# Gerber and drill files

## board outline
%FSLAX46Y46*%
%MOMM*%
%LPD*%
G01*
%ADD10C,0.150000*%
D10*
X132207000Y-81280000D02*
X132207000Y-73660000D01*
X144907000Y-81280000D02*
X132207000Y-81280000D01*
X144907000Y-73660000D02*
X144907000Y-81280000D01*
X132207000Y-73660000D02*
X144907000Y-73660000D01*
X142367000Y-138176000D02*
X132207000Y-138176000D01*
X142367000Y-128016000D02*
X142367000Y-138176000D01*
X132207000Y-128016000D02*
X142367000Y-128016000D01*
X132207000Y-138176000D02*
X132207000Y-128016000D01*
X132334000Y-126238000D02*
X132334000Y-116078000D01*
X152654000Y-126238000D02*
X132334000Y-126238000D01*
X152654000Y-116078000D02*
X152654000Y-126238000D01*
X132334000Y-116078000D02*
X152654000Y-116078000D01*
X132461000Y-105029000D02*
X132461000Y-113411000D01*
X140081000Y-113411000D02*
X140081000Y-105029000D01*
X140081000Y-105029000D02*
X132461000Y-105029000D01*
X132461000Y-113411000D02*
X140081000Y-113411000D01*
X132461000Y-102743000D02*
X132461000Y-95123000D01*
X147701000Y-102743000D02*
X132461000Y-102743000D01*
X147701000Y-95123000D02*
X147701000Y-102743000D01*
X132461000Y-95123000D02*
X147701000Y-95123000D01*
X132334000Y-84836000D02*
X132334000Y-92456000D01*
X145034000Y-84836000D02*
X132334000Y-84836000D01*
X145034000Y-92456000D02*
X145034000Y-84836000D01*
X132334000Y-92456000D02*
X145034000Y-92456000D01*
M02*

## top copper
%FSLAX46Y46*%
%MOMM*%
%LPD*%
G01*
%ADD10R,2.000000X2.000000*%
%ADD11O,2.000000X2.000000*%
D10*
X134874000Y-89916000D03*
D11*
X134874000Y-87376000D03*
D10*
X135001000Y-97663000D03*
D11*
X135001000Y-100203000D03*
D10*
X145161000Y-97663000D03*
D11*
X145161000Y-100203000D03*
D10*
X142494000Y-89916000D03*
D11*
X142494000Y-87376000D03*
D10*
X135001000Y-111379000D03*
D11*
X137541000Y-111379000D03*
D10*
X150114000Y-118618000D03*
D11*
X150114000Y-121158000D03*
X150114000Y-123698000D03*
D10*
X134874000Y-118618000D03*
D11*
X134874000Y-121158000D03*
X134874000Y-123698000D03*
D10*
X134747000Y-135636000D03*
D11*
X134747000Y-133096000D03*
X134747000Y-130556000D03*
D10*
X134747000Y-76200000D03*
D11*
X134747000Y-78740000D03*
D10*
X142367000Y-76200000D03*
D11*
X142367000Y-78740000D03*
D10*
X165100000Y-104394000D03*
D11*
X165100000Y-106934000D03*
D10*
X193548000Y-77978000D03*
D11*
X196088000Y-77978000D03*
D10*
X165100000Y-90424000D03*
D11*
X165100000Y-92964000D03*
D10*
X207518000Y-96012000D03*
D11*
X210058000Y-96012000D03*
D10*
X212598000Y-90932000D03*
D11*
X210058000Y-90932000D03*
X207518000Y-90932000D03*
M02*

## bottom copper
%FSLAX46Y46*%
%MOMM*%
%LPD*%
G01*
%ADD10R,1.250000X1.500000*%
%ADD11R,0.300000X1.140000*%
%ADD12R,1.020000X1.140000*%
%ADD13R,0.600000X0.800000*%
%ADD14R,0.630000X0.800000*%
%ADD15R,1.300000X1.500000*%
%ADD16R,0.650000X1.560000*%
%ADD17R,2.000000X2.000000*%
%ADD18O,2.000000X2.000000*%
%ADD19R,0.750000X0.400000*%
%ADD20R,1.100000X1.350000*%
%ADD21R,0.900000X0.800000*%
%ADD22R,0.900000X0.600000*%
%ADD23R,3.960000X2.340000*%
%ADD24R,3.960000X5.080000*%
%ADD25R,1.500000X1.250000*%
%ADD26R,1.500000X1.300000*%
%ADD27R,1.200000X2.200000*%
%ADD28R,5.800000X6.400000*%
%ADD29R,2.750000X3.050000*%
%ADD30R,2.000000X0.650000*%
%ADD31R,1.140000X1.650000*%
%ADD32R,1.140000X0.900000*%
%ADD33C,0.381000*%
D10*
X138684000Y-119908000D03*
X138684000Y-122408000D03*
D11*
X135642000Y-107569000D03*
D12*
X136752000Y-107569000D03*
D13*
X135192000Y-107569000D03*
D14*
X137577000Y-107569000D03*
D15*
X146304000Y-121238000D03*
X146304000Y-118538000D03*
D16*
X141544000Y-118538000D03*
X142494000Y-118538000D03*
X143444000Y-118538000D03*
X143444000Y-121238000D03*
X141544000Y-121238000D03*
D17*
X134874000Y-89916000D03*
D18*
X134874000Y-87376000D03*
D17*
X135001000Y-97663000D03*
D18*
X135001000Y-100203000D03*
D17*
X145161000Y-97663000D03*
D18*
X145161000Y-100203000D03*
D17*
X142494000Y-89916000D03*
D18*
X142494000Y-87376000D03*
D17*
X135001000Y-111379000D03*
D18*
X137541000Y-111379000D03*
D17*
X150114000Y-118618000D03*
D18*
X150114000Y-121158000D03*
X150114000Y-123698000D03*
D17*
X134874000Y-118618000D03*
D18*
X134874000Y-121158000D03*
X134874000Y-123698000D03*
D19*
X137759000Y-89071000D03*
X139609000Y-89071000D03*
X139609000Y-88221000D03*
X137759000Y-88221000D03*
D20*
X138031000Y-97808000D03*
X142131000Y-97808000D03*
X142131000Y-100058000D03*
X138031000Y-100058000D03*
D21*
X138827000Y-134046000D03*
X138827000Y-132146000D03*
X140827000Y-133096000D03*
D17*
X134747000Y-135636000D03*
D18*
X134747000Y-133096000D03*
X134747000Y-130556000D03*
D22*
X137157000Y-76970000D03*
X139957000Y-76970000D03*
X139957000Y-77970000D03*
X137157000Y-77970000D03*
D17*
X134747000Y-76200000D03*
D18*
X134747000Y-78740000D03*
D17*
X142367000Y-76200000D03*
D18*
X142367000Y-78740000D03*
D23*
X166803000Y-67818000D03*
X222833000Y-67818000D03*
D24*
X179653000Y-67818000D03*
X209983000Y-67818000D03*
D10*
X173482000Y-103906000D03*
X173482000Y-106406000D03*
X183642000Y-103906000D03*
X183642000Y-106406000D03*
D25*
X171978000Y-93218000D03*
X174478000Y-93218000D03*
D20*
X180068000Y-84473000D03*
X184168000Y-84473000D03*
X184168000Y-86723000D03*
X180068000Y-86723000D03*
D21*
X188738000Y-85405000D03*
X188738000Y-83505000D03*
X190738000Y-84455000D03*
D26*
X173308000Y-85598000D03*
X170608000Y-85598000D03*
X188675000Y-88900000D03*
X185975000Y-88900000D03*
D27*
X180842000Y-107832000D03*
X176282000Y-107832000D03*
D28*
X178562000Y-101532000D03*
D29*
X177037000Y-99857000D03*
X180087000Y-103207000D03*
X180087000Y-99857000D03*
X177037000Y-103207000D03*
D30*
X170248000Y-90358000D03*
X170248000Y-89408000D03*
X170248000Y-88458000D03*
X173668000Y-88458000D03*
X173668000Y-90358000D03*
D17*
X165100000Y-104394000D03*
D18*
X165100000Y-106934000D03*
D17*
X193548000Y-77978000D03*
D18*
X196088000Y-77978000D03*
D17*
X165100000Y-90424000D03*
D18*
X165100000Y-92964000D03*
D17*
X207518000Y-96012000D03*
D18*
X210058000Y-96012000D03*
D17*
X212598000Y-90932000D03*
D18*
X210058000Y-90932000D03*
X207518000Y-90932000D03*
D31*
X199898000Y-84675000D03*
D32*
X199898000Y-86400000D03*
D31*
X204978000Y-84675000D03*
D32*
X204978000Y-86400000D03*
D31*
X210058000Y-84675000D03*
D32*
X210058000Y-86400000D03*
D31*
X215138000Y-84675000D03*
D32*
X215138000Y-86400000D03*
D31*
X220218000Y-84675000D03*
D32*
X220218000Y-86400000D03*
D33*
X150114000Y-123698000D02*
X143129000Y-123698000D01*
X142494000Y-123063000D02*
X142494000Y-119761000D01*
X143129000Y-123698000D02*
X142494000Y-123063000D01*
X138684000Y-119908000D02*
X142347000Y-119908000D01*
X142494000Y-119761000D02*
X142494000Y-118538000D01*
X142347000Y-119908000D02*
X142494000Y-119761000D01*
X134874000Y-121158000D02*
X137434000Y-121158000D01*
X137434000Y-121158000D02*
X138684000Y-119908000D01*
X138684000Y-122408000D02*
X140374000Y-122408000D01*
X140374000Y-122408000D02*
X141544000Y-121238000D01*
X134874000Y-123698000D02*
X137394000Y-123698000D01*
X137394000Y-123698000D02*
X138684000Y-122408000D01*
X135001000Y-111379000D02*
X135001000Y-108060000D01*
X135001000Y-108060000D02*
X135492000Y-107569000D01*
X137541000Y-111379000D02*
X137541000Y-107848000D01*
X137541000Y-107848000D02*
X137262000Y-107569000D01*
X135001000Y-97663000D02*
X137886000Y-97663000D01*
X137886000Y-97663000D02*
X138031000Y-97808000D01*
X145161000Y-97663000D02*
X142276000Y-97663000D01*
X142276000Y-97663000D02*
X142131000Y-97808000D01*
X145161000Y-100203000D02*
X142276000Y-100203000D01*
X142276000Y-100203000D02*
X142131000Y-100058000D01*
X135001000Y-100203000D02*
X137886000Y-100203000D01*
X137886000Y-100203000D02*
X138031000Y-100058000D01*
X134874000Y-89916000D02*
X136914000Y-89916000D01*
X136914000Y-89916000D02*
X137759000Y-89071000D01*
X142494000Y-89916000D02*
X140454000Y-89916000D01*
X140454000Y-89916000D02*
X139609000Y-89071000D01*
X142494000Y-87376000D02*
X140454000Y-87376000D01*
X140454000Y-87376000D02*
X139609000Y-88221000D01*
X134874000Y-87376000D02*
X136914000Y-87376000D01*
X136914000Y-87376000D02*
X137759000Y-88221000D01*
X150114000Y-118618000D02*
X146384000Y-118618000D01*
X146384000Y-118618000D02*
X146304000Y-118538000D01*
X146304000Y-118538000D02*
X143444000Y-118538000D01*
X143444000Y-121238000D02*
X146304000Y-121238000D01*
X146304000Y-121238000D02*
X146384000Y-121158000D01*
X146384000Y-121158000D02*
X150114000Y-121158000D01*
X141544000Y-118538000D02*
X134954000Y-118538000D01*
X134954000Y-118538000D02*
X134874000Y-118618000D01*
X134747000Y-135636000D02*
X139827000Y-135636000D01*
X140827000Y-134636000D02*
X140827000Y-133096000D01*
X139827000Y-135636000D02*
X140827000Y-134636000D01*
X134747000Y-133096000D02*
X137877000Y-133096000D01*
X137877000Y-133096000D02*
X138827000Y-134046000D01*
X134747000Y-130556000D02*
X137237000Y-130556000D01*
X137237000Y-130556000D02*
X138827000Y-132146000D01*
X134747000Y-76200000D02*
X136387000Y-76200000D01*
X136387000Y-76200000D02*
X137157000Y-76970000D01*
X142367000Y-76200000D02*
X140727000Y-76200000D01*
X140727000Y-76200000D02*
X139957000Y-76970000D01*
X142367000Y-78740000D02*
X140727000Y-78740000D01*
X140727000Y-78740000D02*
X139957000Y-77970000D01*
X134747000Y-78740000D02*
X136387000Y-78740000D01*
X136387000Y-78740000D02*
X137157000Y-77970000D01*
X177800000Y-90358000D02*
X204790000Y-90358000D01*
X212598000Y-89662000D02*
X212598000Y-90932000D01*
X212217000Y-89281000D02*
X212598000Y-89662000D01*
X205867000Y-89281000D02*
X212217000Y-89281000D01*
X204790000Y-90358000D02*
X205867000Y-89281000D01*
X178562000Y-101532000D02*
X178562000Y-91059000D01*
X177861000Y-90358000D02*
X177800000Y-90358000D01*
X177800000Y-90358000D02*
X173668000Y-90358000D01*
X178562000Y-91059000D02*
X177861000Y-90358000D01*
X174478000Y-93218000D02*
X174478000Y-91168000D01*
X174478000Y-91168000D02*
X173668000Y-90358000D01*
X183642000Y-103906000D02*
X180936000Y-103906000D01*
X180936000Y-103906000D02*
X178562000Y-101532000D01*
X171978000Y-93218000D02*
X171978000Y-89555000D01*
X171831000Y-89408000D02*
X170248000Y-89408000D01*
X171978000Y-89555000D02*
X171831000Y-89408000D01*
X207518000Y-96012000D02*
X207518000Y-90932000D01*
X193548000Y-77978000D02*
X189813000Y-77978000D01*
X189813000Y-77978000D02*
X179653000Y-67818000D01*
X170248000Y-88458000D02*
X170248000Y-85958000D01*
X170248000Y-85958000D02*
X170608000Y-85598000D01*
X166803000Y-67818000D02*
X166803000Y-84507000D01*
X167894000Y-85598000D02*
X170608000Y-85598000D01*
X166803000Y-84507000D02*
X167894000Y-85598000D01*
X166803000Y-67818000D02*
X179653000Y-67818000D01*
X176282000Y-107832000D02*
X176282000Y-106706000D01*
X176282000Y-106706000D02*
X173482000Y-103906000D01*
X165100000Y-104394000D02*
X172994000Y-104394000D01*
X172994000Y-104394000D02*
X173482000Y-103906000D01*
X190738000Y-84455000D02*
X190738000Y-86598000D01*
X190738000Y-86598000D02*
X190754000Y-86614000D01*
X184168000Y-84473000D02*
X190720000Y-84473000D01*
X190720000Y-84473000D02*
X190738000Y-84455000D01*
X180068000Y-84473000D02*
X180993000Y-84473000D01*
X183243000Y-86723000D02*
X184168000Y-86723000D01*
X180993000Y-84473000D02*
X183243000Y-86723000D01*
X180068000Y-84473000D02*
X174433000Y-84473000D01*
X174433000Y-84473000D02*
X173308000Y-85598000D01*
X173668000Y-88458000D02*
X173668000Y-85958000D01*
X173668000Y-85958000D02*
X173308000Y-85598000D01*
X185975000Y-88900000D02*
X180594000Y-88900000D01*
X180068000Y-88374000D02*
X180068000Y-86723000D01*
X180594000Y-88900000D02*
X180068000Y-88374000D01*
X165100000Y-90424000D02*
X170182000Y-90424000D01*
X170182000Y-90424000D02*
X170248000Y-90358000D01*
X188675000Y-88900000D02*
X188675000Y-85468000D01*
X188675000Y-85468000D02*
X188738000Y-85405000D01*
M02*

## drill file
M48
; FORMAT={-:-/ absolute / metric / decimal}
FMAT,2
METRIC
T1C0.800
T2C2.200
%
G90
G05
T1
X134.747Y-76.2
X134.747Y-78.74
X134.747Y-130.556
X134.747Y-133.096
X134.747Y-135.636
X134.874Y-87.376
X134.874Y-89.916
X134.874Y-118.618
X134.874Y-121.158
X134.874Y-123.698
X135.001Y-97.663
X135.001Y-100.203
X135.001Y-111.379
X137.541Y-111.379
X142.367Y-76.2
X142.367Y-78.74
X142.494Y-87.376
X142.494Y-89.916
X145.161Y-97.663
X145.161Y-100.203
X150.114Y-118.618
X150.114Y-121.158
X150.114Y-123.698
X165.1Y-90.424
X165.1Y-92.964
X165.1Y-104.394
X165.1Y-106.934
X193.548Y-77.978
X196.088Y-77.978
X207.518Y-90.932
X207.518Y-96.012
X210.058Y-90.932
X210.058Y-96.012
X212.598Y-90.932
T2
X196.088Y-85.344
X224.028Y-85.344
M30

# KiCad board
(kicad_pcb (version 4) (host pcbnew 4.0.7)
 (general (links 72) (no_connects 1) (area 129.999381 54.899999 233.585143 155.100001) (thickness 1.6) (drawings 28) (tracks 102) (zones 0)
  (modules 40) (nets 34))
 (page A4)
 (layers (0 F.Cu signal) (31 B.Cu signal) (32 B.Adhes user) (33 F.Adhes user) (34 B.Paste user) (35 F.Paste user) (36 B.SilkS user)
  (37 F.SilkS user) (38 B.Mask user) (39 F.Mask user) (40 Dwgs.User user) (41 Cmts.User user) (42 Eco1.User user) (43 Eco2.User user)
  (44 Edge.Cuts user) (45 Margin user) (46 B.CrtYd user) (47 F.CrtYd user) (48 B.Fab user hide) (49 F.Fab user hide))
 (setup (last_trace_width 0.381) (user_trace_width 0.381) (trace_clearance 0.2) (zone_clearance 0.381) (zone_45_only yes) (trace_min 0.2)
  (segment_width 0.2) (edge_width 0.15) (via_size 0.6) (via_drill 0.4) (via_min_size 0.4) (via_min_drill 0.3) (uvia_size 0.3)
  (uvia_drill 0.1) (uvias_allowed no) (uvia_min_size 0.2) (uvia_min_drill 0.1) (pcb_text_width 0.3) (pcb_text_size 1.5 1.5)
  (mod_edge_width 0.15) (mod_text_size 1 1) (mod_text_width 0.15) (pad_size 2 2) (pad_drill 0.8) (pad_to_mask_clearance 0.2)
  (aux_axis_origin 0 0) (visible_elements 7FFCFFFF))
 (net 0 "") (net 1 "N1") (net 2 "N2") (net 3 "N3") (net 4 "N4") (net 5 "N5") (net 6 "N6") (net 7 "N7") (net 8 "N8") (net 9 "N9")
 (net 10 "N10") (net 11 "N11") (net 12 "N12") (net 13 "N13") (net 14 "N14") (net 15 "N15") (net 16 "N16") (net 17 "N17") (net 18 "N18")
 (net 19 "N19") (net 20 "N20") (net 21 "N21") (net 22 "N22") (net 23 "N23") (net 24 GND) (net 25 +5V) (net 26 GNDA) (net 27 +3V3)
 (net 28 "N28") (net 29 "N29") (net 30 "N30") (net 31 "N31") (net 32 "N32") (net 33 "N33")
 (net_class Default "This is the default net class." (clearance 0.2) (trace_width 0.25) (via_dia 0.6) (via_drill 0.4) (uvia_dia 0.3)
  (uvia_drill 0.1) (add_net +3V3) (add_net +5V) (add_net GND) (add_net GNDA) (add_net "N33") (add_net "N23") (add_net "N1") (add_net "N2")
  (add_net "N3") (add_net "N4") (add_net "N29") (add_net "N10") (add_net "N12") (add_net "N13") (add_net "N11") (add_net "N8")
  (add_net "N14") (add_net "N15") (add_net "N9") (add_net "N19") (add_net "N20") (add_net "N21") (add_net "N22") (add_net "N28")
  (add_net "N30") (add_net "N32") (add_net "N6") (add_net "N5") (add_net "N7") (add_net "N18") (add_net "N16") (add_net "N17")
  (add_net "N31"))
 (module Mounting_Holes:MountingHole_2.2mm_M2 (layer F.Cu) (at 224.028 85.344)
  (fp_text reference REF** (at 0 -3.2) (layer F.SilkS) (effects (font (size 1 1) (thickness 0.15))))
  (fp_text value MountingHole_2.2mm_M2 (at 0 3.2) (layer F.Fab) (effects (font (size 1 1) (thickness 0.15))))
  (pad 1 np_thru_hole circle (at 0 0) (size 2.2 2.2) (drill 2.2) (layers *.Cu *.Mask)))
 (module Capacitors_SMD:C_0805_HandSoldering (layer B.Cu) (at 138.684 121.158 270)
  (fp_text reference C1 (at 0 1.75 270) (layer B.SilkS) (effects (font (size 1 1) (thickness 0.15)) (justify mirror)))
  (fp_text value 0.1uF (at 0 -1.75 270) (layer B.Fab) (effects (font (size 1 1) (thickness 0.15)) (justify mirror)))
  (pad 1 smd rect (at -1.25 0 270) (size 1.5 1.25) (layers B.Cu B.Paste B.Mask) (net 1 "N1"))
  (pad 2 smd rect (at 1.25 0 270) (size 1.5 1.25) (layers B.Cu B.Paste B.Mask) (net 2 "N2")))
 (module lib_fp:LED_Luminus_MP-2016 (layer B.Cu) (at 136.017 107.569)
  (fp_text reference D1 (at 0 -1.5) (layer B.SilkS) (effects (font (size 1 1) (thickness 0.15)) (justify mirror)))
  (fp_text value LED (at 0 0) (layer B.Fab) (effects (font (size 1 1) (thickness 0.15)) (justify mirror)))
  (pad 1 smd rect (at -0.225 0) (size 0.3 1.14) (drill (offset -0.15 0)) (layers B.Cu B.Paste B.Mask) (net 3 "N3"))
  (pad 2 smd rect (at 0.225 0) (size 1.02 1.14) (drill (offset 0.51 0)) (layers B.Cu B.Paste B.Mask) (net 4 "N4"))
  (pad 1 smd rect (at -0.525 0) (size 0.6 0.8) (drill (offset -0.3 0)) (layers B.Cu B.Paste B.Mask) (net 3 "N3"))
  (pad 2 smd rect (at 1.245 0) (size 0.63 0.8) (drill (offset 0.315 0)) (layers B.Cu B.Paste B.Mask) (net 4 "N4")))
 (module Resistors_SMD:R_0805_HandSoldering (layer B.Cu) (at 146.304 119.888 90)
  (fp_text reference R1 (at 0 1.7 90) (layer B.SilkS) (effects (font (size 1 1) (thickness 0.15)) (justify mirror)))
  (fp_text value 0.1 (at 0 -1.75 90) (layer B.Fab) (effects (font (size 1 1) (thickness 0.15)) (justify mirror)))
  (pad 1 smd rect (at -1.35 0 90) (size 1.5 1.3) (layers B.Cu B.Paste B.Mask) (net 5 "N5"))
  (pad 2 smd rect (at 1.35 0 90) (size 1.5 1.3) (layers B.Cu B.Paste B.Mask) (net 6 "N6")))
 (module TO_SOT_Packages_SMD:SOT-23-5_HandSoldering (layer B.Cu) (at 142.494 119.888 270)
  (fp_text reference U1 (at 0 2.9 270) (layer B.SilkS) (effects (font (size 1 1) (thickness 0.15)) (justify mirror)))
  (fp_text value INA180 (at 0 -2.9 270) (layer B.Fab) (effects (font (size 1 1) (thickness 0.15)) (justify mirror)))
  (pad 1 smd rect (at -1.35 0.95 270) (size 1.56 0.65) (layers B.Cu B.Paste B.Mask) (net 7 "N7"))
  (pad 2 smd rect (at -1.35 0 270) (size 1.56 0.65) (layers B.Cu B.Paste B.Mask) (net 1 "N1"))
  (pad 3 smd rect (at -1.35 -0.95 270) (size 1.56 0.65) (layers B.Cu B.Paste B.Mask) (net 6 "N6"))
  (pad 4 smd rect (at 1.35 -0.95 270) (size 1.56 0.65) (layers B.Cu B.Paste B.Mask) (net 5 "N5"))
  (pad 5 smd rect (at 1.35 0.95 270) (size 1.56 0.65) (layers B.Cu B.Paste B.Mask) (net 2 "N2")))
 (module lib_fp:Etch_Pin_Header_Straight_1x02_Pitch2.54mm (layer F.Cu) (at 134.874 89.916 180)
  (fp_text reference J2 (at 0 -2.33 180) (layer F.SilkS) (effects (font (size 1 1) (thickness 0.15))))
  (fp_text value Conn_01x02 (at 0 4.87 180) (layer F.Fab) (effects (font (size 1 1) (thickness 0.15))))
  (pad 1 thru_hole rect (at 0 0 180) (size 2 2) (drill 0.8) (layers *.Cu *.Mask) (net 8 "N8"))
  (pad 2 thru_hole oval (at 0 2.54 180) (size 2 2) (drill 0.8) (layers *.Cu *.Mask) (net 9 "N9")))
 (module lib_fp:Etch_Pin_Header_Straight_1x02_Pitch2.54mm (layer F.Cu) (at 135.001 97.663)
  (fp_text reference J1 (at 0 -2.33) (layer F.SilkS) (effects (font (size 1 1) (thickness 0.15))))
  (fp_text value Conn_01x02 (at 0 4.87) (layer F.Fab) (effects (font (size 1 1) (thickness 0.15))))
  (pad 1 thru_hole rect (at 0 0) (size 2 2) (drill 0.8) (layers *.Cu *.Mask) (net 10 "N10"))
  (pad 2 thru_hole oval (at 0 2.54) (size 2 2) (drill 0.8) (layers *.Cu *.Mask) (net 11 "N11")))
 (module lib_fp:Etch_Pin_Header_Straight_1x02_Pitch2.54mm (layer F.Cu) (at 145.161 97.663)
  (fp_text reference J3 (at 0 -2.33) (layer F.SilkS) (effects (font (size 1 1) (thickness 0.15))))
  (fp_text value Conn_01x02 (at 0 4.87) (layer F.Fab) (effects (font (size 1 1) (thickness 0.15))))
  (pad 1 thru_hole rect (at 0 0) (size 2 2) (drill 0.8) (layers *.Cu *.Mask) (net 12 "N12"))
  (pad 2 thru_hole oval (at 0 2.54) (size 2 2) (drill 0.8) (layers *.Cu *.Mask) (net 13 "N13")))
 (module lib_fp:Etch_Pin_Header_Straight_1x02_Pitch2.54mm (layer F.Cu) (at 142.494 89.916 180)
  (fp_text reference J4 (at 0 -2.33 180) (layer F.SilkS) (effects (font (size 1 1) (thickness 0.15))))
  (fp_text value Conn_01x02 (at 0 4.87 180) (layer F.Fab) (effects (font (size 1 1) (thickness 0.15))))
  (pad 1 thru_hole rect (at 0 0 180) (size 2 2) (drill 0.8) (layers *.Cu *.Mask) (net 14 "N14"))
  (pad 2 thru_hole oval (at 0 2.54 180) (size 2 2) (drill 0.8) (layers *.Cu *.Mask) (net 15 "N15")))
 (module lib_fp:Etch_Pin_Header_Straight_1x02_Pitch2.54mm (layer F.Cu) (at 135.001 111.379 90)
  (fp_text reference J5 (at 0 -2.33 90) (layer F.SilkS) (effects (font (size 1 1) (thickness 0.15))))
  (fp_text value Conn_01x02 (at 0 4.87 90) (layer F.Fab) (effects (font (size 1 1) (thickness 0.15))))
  (pad 1 thru_hole rect (at 0 0 90) (size 2 2) (drill 0.8) (layers *.Cu *.Mask) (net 3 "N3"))
  (pad 2 thru_hole oval (at 0 2.54 90) (size 2 2) (drill 0.8) (layers *.Cu *.Mask) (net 4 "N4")))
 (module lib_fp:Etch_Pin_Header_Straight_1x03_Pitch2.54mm (layer F.Cu) (at 150.114 118.618)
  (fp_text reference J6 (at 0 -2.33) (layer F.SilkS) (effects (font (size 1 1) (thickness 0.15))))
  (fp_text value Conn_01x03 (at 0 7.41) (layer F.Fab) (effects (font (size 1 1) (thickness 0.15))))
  (pad 1 thru_hole rect (at 0 0) (size 2 2) (drill 0.8) (layers *.Cu *.Mask) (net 6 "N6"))
  (pad 2 thru_hole oval (at 0 2.54) (size 2 2) (drill 0.8) (layers *.Cu *.Mask) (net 5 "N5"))
  (pad 3 thru_hole oval (at 0 5.08) (size 2 2) (drill 0.8) (layers *.Cu *.Mask) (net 1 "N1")))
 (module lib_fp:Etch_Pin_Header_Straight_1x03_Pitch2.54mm (layer F.Cu) (at 134.874 118.618)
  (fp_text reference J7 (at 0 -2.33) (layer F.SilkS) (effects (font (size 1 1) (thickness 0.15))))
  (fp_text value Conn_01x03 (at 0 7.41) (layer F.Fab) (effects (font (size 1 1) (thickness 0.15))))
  (pad 1 thru_hole rect (at 0 0) (size 2 2) (drill 0.8) (layers *.Cu *.Mask) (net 7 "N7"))
  (pad 2 thru_hole oval (at 0 2.54) (size 2 2) (drill 0.8) (layers *.Cu *.Mask) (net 1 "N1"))
  (pad 3 thru_hole oval (at 0 5.08) (size 2 2) (drill 0.8) (layers *.Cu *.Mask) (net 2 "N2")))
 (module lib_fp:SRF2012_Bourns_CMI (layer B.Cu) (at 138.684 88.646)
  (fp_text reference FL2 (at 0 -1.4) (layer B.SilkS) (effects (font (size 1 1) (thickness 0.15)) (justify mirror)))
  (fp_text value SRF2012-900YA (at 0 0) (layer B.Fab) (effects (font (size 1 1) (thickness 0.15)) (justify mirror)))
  (pad 1 smd rect (at -0.925 0.425) (size 0.75 0.4) (layers B.Cu B.Paste B.Mask) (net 8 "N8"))
  (pad 2 smd rect (at 0.925 0.425) (size 0.75 0.4) (layers B.Cu B.Paste B.Mask) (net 14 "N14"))
  (pad 3 smd rect (at 0.925 -0.425) (size 0.75 0.4) (layers B.Cu B.Paste B.Mask) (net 15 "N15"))
  (pad 4 smd rect (at -0.925 -0.425) (size 0.75 0.4) (layers B.Cu B.Paste B.Mask) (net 9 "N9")))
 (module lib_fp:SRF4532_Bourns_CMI (layer B.Cu) (at 140.081 98.933)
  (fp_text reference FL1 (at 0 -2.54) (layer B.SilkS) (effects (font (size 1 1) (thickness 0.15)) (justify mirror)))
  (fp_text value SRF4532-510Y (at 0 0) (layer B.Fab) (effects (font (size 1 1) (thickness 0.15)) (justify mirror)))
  (pad 1 smd rect (at -2.05 -1.125) (size 1.1 1.35) (layers B.Cu B.Paste B.Mask) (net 10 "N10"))
  (pad 2 smd rect (at 2.05 -1.125) (size 1.1 1.35) (layers B.Cu B.Paste B.Mask) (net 12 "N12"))
  (pad 3 smd rect (at 2.05 1.125) (size 1.1 1.35) (layers B.Cu B.Paste B.Mask) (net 13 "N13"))
  (pad 4 smd rect (at -2.05 1.125) (size 1.1 1.35) (layers B.Cu B.Paste B.Mask) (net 11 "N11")))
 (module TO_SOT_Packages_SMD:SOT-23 (layer B.Cu) (at 139.827 133.096)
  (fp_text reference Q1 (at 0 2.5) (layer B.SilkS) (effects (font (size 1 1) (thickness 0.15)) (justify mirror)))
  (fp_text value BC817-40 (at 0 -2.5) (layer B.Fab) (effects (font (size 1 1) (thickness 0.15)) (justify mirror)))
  (pad 1 smd rect (at -1 0.95) (size 0.9 0.8) (layers B.Cu B.Paste B.Mask) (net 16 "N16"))
  (pad 2 smd rect (at -1 -0.95) (size 0.9 0.8) (layers B.Cu B.Paste B.Mask) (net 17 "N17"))
  (pad 3 smd rect (at 1 0) (size 0.9 0.8) (layers B.Cu B.Paste B.Mask) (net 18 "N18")))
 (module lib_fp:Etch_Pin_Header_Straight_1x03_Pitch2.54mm (layer F.Cu) (at 134.747 135.636 180)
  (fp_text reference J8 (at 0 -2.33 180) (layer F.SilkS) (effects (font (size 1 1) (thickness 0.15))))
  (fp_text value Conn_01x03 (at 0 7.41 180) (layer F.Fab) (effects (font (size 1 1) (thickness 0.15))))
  (pad 1 thru_hole rect (at 0 0 180) (size 2 2) (drill 0.8) (layers *.Cu *.Mask) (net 18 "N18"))
  (pad 2 thru_hole oval (at 0 2.54 180) (size 2 2) (drill 0.8) (layers *.Cu *.Mask) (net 16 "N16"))
  (pad 3 thru_hole oval (at 0 5.08 180) (size 2 2) (drill 0.8) (layers *.Cu *.Mask) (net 17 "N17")))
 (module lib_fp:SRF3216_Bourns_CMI (layer B.Cu) (at 138.557 77.47)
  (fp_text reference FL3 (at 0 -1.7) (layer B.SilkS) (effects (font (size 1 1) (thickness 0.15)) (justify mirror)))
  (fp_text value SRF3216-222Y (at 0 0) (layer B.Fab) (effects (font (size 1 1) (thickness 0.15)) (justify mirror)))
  (pad 1 smd rect (at -1.4 -0.5) (size 0.9 0.6) (layers B.Cu B.Paste B.Mask) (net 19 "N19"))
  (pad 2 smd rect (at 1.4 -0.5) (size 0.9 0.6) (layers B.Cu B.Paste B.Mask) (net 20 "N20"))
  (pad 3 smd rect (at 1.4 0.5) (size 0.9 0.6) (layers B.Cu B.Paste B.Mask) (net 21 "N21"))
  (pad 4 smd rect (at -1.4 0.5) (size 0.9 0.6) (layers B.Cu B.Paste B.Mask) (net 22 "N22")))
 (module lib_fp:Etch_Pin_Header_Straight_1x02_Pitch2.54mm (layer F.Cu) (at 134.747 76.2)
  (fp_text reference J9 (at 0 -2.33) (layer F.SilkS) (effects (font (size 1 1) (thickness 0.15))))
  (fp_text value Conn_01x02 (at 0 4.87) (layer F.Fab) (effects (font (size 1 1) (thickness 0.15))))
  (pad 1 thru_hole rect (at 0 0) (size 2 2) (drill 0.8) (layers *.Cu *.Mask) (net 19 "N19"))
  (pad 2 thru_hole oval (at 0 2.54) (size 2 2) (drill 0.8) (layers *.Cu *.Mask) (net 22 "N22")))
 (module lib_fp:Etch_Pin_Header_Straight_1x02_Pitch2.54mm (layer F.Cu) (at 142.367 76.2)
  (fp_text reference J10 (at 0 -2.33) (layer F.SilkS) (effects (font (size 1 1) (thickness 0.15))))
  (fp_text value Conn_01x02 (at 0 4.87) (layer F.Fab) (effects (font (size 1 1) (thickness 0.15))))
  (pad 1 thru_hole rect (at 0 0) (size 2 2) (drill 0.8) (layers *.Cu *.Mask) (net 20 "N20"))
  (pad 2 thru_hole oval (at 0 2.54) (size 2 2) (drill 0.8) (layers *.Cu *.Mask) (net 21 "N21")))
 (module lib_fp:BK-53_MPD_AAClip (layer B.Cu) (at 194.818 67.818 270)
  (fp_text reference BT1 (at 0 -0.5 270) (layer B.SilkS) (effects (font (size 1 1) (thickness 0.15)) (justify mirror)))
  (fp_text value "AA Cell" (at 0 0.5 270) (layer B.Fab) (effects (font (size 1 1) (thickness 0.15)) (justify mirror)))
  (pad 1 smd rect (at 0 28.015 270) (size 2.34 3.96) (layers B.Cu B.Paste B.Mask) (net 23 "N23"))
  (pad 2 smd rect (at 0 -28.015 270) (size 2.34 3.96) (layers B.Cu B.Paste B.Mask) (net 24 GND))
  (pad 1 smd rect (at 0 15.165 270) (size 5.08 3.96) (layers B.Cu B.Paste B.Mask) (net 23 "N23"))
  (pad 2 smd rect (at 0 -15.165 270) (size 5.08 3.96) (layers B.Cu B.Paste B.Mask) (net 24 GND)))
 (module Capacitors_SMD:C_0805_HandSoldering (layer B.Cu) (at 173.482 105.156 270)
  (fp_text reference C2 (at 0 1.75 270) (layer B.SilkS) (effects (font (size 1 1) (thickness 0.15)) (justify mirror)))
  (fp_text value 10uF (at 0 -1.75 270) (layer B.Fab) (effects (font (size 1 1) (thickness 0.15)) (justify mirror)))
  (pad 1 smd rect (at -1.25 0 270) (size 1.5 1.25) (layers B.Cu B.Paste B.Mask) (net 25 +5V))
  (pad 2 smd rect (at 1.25 0 270) (size 1.5 1.25) (layers B.Cu B.Paste B.Mask) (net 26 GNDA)))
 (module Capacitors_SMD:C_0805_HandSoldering (layer B.Cu) (at 183.642 105.156 270)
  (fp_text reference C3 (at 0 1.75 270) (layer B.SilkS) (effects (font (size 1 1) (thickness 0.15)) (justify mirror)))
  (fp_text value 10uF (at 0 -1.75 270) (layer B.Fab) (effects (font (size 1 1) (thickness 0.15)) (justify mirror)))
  (pad 1 smd rect (at -1.25 0 270) (size 1.5 1.25) (layers B.Cu B.Paste B.Mask) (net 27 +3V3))
  (pad 2 smd rect (at 1.25 0 270) (size 1.5 1.25) (layers B.Cu B.Paste B.Mask) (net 26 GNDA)))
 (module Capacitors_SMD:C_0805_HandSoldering (layer B.Cu) (at 173.228 93.218)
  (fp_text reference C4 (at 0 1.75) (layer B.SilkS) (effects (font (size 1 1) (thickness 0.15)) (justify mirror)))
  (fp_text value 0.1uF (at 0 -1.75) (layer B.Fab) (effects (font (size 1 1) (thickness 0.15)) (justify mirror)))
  (pad 1 smd rect (at -1.25 0) (size 1.5 1.25) (layers B.Cu B.Paste B.Mask) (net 26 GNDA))
  (pad 2 smd rect (at 1.25 0) (size 1.5 1.25) (layers B.Cu B.Paste B.Mask) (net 27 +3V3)))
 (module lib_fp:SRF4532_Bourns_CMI (layer B.Cu) (at 182.118 85.598)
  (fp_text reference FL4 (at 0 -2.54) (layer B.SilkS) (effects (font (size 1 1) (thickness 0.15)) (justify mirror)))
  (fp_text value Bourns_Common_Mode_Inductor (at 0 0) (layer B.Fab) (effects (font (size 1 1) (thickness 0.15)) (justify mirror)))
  (pad 1 smd rect (at -2.05 -1.125) (size 1.1 1.35) (layers B.Cu B.Paste B.Mask) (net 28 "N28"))
  (pad 2 smd rect (at 2.05 -1.125) (size 1.1 1.35) (layers B.Cu B.Paste B.Mask) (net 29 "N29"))
  (pad 3 smd rect (at 2.05 1.125) (size 1.1 1.35) (layers B.Cu B.Paste B.Mask) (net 28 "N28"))
  (pad 4 smd rect (at -2.05 1.125) (size 1.1 1.35) (layers B.Cu B.Paste B.Mask) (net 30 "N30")))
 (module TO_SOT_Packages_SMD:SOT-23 (layer B.Cu) (at 189.738 84.455)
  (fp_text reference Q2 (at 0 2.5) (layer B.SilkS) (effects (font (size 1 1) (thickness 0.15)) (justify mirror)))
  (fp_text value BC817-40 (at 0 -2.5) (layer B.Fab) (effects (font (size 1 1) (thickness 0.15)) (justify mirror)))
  (pad 1 smd rect (at -1 0.95) (size 0.9 0.8) (layers B.Cu B.Paste B.Mask) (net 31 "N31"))
  (pad 2 smd rect (at -1 -0.95) (size 0.9 0.8) (layers B.Cu B.Paste B.Mask) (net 24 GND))
  (pad 3 smd rect (at 1 0) (size 0.9 0.8) (layers B.Cu B.Paste B.Mask) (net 29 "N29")))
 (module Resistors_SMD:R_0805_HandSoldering (layer B.Cu) (at 171.958 85.598 180)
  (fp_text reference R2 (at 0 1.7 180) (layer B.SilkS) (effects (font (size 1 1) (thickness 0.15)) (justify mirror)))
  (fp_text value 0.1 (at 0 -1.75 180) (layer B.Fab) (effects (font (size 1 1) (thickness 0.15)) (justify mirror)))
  (pad 1 smd rect (at -1.35 0 180) (size 1.5 1.3) (layers B.Cu B.Paste B.Mask) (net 28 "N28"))
  (pad 2 smd rect (at 1.35 0 180) (size 1.5 1.3) (layers B.Cu B.Paste B.Mask) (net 23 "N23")))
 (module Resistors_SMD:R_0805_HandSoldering (layer B.Cu) (at 187.325 88.9 180)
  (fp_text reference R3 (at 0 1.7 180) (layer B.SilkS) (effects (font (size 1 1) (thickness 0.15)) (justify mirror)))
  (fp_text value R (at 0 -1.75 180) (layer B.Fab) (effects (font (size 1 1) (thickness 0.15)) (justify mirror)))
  (pad 1 smd rect (at -1.35 0 180) (size 1.5 1.3) (layers B.Cu B.Paste B.Mask) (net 31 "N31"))
  (pad 2 smd rect (at 1.35 0 180) (size 1.5 1.3) (layers B.Cu B.Paste B.Mask) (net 30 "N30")))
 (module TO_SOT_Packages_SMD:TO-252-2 (layer B.Cu) (at 178.562 103.632 90)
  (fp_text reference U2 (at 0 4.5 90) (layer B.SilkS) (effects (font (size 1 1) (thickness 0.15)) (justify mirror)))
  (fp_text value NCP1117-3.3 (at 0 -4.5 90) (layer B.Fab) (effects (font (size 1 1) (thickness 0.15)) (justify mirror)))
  (pad 1 smd rect (at -4.2 2.28 90) (size 2.2 1.2) (layers B.Cu B.Paste B.Mask) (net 26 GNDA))
  (pad 3 smd rect (at -4.2 -2.28 90) (size 2.2 1.2) (layers B.Cu B.Paste B.Mask) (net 25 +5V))
  (pad 2 smd rect (at 2.1 0 90) (size 6.4 5.8) (layers B.Cu B.Mask) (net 27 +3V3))
  (pad 2 smd rect (at 3.775 -1.525 90) (size 3.05 2.75) (layers B.Cu B.Paste) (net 27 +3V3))
  (pad 2 smd rect (at 0.425 1.525 90) (size 3.05 2.75) (layers B.Cu B.Paste) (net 27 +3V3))
  (pad 2 smd rect (at 3.775 1.525 90) (size 3.05 2.75) (layers B.Cu B.Paste) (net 27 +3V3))
  (pad 2 smd rect (at 0.425 -1.525 90) (size 3.05 2.75) (layers B.Cu B.Paste) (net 27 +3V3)))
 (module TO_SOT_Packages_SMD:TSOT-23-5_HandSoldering (layer B.Cu) (at 171.958 89.408)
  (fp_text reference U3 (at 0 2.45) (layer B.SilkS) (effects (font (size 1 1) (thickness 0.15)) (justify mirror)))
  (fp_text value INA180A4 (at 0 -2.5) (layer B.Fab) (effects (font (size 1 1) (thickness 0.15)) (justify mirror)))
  (pad 1 smd rect (at -1.71 0.95) (size 2 0.65) (layers B.Cu B.Paste B.Mask) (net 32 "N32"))
  (pad 2 smd rect (at -1.71 0) (size 2 0.65) (layers B.Cu B.Paste B.Mask) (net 26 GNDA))
  (pad 3 smd rect (at -1.71 -0.95) (size 2 0.65) (layers B.Cu B.Paste B.Mask) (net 23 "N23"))
  (pad 4 smd rect (at 1.71 -0.95) (size 2 0.65) (layers B.Cu B.Paste B.Mask) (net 28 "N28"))
  (pad 5 smd rect (at 1.71 0.95) (size 2 0.65) (layers B.Cu B.Paste B.Mask) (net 27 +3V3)))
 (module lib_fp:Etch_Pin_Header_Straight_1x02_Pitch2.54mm (layer F.Cu) (at 165.1 104.394)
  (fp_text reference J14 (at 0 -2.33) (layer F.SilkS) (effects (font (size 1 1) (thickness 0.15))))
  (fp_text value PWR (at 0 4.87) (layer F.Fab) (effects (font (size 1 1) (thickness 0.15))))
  (pad 1 thru_hole rect (at 0 0) (size 2 2) (drill 0.8) (layers *.Cu *.Mask) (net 25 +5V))
  (pad 2 thru_hole oval (at 0 2.54) (size 2 2) (drill 0.8) (layers *.Cu *.Mask) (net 26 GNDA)))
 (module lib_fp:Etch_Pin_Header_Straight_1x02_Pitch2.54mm (layer F.Cu) (at 193.548 77.978 90)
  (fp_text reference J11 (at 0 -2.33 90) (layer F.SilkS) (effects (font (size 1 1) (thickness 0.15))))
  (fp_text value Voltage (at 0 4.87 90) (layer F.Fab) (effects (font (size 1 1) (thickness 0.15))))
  (pad 1 thru_hole rect (at 0 0 90) (size 2 2) (drill 0.8) (layers *.Cu *.Mask) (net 23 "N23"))
  (pad 2 thru_hole oval (at 0 2.54 90) (size 2 2) (drill 0.8) (layers *.Cu *.Mask) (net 24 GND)))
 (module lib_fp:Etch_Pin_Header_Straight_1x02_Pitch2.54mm (layer F.Cu) (at 165.1 90.424)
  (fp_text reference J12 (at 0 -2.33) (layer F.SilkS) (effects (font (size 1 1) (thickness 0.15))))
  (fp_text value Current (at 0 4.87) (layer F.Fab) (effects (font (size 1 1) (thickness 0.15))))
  (pad 1 thru_hole rect (at 0 0) (size 2 2) (drill 0.8) (layers *.Cu *.Mask) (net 32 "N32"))
  (pad 2 thru_hole oval (at 0 2.54) (size 2 2) (drill 0.8) (layers *.Cu *.Mask) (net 26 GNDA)))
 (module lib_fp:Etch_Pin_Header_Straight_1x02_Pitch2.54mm (layer F.Cu) (at 207.518 96.012 90)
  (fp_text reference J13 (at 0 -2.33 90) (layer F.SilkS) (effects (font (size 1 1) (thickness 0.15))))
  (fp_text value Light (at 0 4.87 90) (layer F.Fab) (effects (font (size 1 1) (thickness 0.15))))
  (pad 1 thru_hole rect (at 0 0 90) (size 2 2) (drill 0.8) (layers *.Cu *.Mask) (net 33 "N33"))
  (pad 2 thru_hole oval (at 0 2.54 90) (size 2 2) (drill 0.8) (layers *.Cu *.Mask) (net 26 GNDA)))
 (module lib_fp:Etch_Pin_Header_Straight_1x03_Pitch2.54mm (layer F.Cu) (at 212.598 90.932 270)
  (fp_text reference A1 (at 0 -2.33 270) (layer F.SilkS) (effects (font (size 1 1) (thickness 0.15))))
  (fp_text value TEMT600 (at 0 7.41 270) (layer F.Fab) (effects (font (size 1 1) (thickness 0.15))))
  (pad 1 thru_hole rect (at 0 0 270) (size 2 2) (drill 0.8) (layers *.Cu *.Mask) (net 27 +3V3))
  (pad 2 thru_hole oval (at 0 2.54 270) (size 2 2) (drill 0.8) (layers *.Cu *.Mask) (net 26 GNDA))
  (pad 3 thru_hole oval (at 0 5.08 270) (size 2 2) (drill 0.8) (layers *.Cu *.Mask) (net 33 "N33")))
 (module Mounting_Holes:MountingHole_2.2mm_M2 (layer F.Cu) (at 196.088 85.344)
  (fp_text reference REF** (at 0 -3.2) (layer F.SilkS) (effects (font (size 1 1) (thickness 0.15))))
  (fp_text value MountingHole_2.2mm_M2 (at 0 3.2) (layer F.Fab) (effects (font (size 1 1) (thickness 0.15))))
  (pad 1 np_thru_hole circle (at 0 0) (size 2.2 2.2) (drill 2.2) (layers *.Cu *.Mask)))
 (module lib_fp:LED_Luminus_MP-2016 (layer B.Cu) (at 199.898 85.725 270)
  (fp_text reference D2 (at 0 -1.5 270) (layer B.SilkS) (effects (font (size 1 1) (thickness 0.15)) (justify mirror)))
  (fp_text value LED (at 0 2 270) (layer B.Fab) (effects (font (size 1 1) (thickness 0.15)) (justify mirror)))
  (pad 1 smd rect (at -1.05 0 270) (size 1.65 1.14) (layers B.Cu B.Paste B.Mask) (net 24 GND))
  (pad 2 smd rect (at 0.675 0 270) (size 0.9 1.14) (layers B.Cu B.Paste B.Mask) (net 29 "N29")))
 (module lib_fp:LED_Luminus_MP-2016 (layer B.Cu) (at 204.978 85.725 270)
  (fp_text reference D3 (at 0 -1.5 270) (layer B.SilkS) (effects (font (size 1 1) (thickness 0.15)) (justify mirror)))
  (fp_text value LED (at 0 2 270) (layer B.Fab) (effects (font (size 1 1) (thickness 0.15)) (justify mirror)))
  (pad 1 smd rect (at -1.05 0 270) (size 1.65 1.14) (layers B.Cu B.Paste B.Mask) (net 24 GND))
  (pad 2 smd rect (at 0.675 0 270) (size 0.9 1.14) (layers B.Cu B.Paste B.Mask) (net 29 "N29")))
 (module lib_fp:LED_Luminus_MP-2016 (layer B.Cu) (at 210.058 85.725 270)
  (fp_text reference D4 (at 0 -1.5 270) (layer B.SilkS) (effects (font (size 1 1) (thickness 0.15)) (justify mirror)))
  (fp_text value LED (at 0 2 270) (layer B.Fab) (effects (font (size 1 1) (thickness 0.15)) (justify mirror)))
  (pad 1 smd rect (at -1.05 0 270) (size 1.65 1.14) (layers B.Cu B.Paste B.Mask) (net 24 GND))
  (pad 2 smd rect (at 0.675 0 270) (size 0.9 1.14) (layers B.Cu B.Paste B.Mask) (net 29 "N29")))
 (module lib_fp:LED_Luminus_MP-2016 (layer B.Cu) (at 215.138 85.725 270)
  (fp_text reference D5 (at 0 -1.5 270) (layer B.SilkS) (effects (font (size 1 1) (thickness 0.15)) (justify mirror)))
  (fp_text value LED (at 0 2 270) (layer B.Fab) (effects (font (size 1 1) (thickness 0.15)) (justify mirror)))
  (pad 1 smd rect (at -1.05 0 270) (size 1.65 1.14) (layers B.Cu B.Paste B.Mask) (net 24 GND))
  (pad 2 smd rect (at 0.675 0 270) (size 0.9 1.14) (layers B.Cu B.Paste B.Mask) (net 29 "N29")))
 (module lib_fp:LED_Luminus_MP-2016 (layer B.Cu) (at 220.218 85.725 270)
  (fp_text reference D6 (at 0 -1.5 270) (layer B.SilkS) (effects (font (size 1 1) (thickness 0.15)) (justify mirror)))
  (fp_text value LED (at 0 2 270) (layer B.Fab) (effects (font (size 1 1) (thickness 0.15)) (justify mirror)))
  (pad 1 smd rect (at -1.05 0 270) (size 1.65 1.14) (layers B.Cu B.Paste B.Mask) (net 24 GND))
  (pad 2 smd rect (at 0.675 0 270) (size 0.9 1.14) (layers B.Cu B.Paste B.Mask) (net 29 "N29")))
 (gr_line (start 132.207 81.28) (end 132.207 73.66) (angle 90) (layer Edge.Cuts) (width 0.15))
 (gr_line (start 144.907 81.28) (end 132.207 81.28) (angle 90) (layer Edge.Cuts) (width 0.15))
 (gr_line (start 144.907 73.66) (end 144.907 81.28) (angle 90) (layer Edge.Cuts) (width 0.15))
 (gr_line (start 132.207 73.66) (end 144.907 73.66) (angle 90) (layer Edge.Cuts) (width 0.15))
 (gr_line (start 142.367 138.176) (end 132.207 138.176) (angle 90) (layer Edge.Cuts) (width 0.15))
 (gr_line (start 142.367 128.016) (end 142.367 138.176) (angle 90) (layer Edge.Cuts) (width 0.15))
 (gr_line (start 132.207 128.016) (end 142.367 128.016) (angle 90) (layer Edge.Cuts) (width 0.15))
 (gr_line (start 132.207 138.176) (end 132.207 128.016) (angle 90) (layer Edge.Cuts) (width 0.15))
 (gr_line (start 132.334 126.238) (end 132.334 116.078) (angle 90) (layer Edge.Cuts) (width 0.15))
 (gr_line (start 152.654 126.238) (end 132.334 126.238) (angle 90) (layer Edge.Cuts) (width 0.15))
 (gr_line (start 152.654 116.078) (end 152.654 126.238) (angle 90) (layer Edge.Cuts) (width 0.15))
 (gr_line (start 132.334 116.078) (end 152.654 116.078) (angle 90) (layer Edge.Cuts) (width 0.15))
 (gr_line (start 132.461 105.029) (end 132.461 113.411) (angle 90) (layer Edge.Cuts) (width 0.15))
 (gr_line (start 140.081 113.411) (end 140.081 105.029) (angle 90) (layer Edge.Cuts) (width 0.15))
 (gr_line (start 140.081 105.029) (end 132.461 105.029) (angle 90) (layer Edge.Cuts) (width 0.15))
 (gr_line (start 132.461 113.411) (end 140.081 113.411) (angle 90) (layer Edge.Cuts) (width 0.15))
 (gr_line (start 132.461 102.743) (end 132.461 95.123) (angle 90) (layer Edge.Cuts) (width 0.15))
 (gr_line (start 147.701 102.743) (end 132.461 102.743) (angle 90) (layer Edge.Cuts) (width 0.15))
 (gr_line (start 147.701 95.123) (end 147.701 102.743) (angle 90) (layer Edge.Cuts) (width 0.15))
 (gr_line (start 132.461 95.123) (end 147.701 95.123) (angle 90) (layer Edge.Cuts) (width 0.15))
 (gr_line (start 132.334 84.836) (end 132.334 92.456) (angle 90) (layer Edge.Cuts) (width 0.15))
 (gr_line (start 145.034 84.836) (end 132.334 84.836) (angle 90) (layer Edge.Cuts) (width 0.15))
 (gr_line (start 145.034 92.456) (end 145.034 84.836) (angle 90) (layer Edge.Cuts) (width 0.15))
 (gr_line (start 132.334 92.456) (end 145.034 92.456) (angle 90) (layer Edge.Cuts) (width 0.15))
 (segment (start 150.114 123.698) (end 143.129 123.698) (width 0.381) (layer B.Cu) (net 1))
 (segment (start 142.494 123.063) (end 142.494 119.761) (width 0.381) (layer B.Cu) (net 1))
 (segment (start 143.129 123.698) (end 142.494 123.063) (width 0.381) (layer B.Cu) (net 1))
 (segment (start 138.684 119.908) (end 142.347 119.908) (width 0.381) (layer B.Cu) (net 1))
 (segment (start 142.494 119.761) (end 142.494 118.538) (width 0.381) (layer B.Cu) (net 1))
 (segment (start 142.347 119.908) (end 142.494 119.761) (width 0.381) (layer B.Cu) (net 1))
 (segment (start 134.874 121.158) (end 137.434 121.158) (width 0.381) (layer B.Cu) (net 1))
 (segment (start 137.434 121.158) (end 138.684 119.908) (width 0.381) (layer B.Cu) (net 1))
 (segment (start 138.684 122.408) (end 140.374 122.408) (width 0.381) (layer B.Cu) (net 2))
 (segment (start 140.374 122.408) (end 141.544 121.238) (width 0.381) (layer B.Cu) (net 2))
 (segment (start 134.874 123.698) (end 137.394 123.698) (width 0.381) (layer B.Cu) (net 2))
 (segment (start 137.394 123.698) (end 138.684 122.408) (width 0.381) (layer B.Cu) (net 2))
 (segment (start 135.001 111.379) (end 135.001 108.06) (width 0.381) (layer B.Cu) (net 3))
 (segment (start 135.001 108.06) (end 135.492 107.569) (width 0.381) (layer B.Cu) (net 3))
 (segment (start 137.541 111.379) (end 137.541 107.848) (width 0.381) (layer B.Cu) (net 4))
 (segment (start 137.541 107.848) (end 137.262 107.569) (width 0.381) (layer B.Cu) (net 4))
 (segment (start 135.001 97.663) (end 137.886 97.663) (width 0.381) (layer B.Cu) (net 10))
 (segment (start 137.886 97.663) (end 138.031 97.808) (width 0.381) (layer B.Cu) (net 10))
 (segment (start 145.161 97.663) (end 142.276 97.663) (width 0.381) (layer B.Cu) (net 12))
 (segment (start 142.276 97.663) (end 142.131 97.808) (width 0.381) (layer B.Cu) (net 12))
 (segment (start 145.161 100.203) (end 142.276 100.203) (width 0.381) (layer B.Cu) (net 13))
 (segment (start 142.276 100.203) (end 142.131 100.058) (width 0.381) (layer B.Cu) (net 13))
 (segment (start 135.001 100.203) (end 137.886 100.203) (width 0.381) (layer B.Cu) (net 11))
 (segment (start 137.886 100.203) (end 138.031 100.058) (width 0.381) (layer B.Cu) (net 11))
 (segment (start 134.874 89.916) (end 136.914 89.916) (width 0.381) (layer B.Cu) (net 8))
 (segment (start 136.914 89.916) (end 137.759 89.071) (width 0.381) (layer B.Cu) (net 8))
 (segment (start 142.494 89.916) (end 140.454 89.916) (width 0.381) (layer B.Cu) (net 14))
 (segment (start 140.454 89.916) (end 139.609 89.071) (width 0.381) (layer B.Cu) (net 14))
 (segment (start 142.494 87.376) (end 140.454 87.376) (width 0.381) (layer B.Cu) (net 15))
 (segment (start 140.454 87.376) (end 139.609 88.221) (width 0.381) (layer B.Cu) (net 15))
 (segment (start 134.874 87.376) (end 136.914 87.376) (width 0.381) (layer B.Cu) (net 9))
 (segment (start 136.914 87.376) (end 137.759 88.221) (width 0.381) (layer B.Cu) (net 9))
 (segment (start 150.114 118.618) (end 146.384 118.618) (width 0.381) (layer B.Cu) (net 6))
 (segment (start 146.384 118.618) (end 146.304 118.538) (width 0.381) (layer B.Cu) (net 6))
 (segment (start 146.304 118.538) (end 143.444 118.538) (width 0.381) (layer B.Cu) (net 6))
 (segment (start 143.444 121.238) (end 146.304 121.238) (width 0.381) (layer B.Cu) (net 5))
 (segment (start 146.304 121.238) (end 146.384 121.158) (width 0.381) (layer B.Cu) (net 5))
 (segment (start 146.384 121.158) (end 150.114 121.158) (width 0.381) (layer B.Cu) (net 5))
 (segment (start 141.544 118.538) (end 134.954 118.538) (width 0.381) (layer B.Cu) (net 7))
 (segment (start 134.954 118.538) (end 134.874 118.618) (width 0.381) (layer B.Cu) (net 7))
 (segment (start 134.747 135.636) (end 139.827 135.636) (width 0.381) (layer B.Cu) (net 18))
 (segment (start 140.827 134.636) (end 140.827 133.096) (width 0.381) (layer B.Cu) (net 18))
 (segment (start 139.827 135.636) (end 140.827 134.636) (width 0.381) (layer B.Cu) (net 18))
 (segment (start 134.747 133.096) (end 137.877 133.096) (width 0.381) (layer B.Cu) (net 16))
 (segment (start 137.877 133.096) (end 138.827 134.046) (width 0.381) (layer B.Cu) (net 16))
 (segment (start 134.747 130.556) (end 137.237 130.556) (width 0.381) (layer B.Cu) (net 17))
 (segment (start 137.237 130.556) (end 138.827 132.146) (width 0.381) (layer B.Cu) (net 17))
 (segment (start 134.747 76.2) (end 136.387 76.2) (width 0.381) (layer B.Cu) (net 19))
 (segment (start 136.387 76.2) (end 137.157 76.97) (width 0.381) (layer B.Cu) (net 19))
 (segment (start 142.367 76.2) (end 140.727 76.2) (width 0.381) (layer B.Cu) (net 20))
 (segment (start 140.727 76.2) (end 139.957 76.97) (width 0.381) (layer B.Cu) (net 20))
 (segment (start 142.367 78.74) (end 140.727 78.74) (width 0.381) (layer B.Cu) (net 21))
 (segment (start 140.727 78.74) (end 139.957 77.97) (width 0.381) (layer B.Cu) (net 21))
 (segment (start 134.747 78.74) (end 136.387 78.74) (width 0.381) (layer B.Cu) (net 22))
 (segment (start 136.387 78.74) (end 137.157 77.97) (width 0.381) (layer B.Cu) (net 22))
 (segment (start 177.8 90.358) (end 204.79 90.358) (width 0.381) (layer B.Cu) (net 27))
 (segment (start 212.598 89.662) (end 212.598 90.932) (width 0.381) (layer B.Cu) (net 27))
 (segment (start 212.217 89.281) (end 212.598 89.662) (width 0.381) (layer B.Cu) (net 27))
 (segment (start 205.867 89.281) (end 212.217 89.281) (width 0.381) (layer B.Cu) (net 27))
 (segment (start 204.79 90.358) (end 205.867 89.281) (width 0.381) (layer B.Cu) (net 27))
 (segment (start 178.562 101.532) (end 178.562 91.059) (width 0.381) (layer B.Cu) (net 27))
 (segment (start 177.861 90.358) (end 177.8 90.358) (width 0.381) (layer B.Cu) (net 27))
 (segment (start 177.8 90.358) (end 173.668 90.358) (width 0.381) (layer B.Cu) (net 27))
 (segment (start 178.562 91.059) (end 177.861 90.358) (width 0.381) (layer B.Cu) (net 27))
 (segment (start 174.478 93.218) (end 174.478 91.168) (width 0.381) (layer B.Cu) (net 27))
 (segment (start 174.478 91.168) (end 173.668 90.358) (width 0.381) (layer B.Cu) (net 27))
 (segment (start 183.642 103.906) (end 180.936 103.906) (width 0.381) (layer B.Cu) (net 27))
 (segment (start 180.936 103.906) (end 178.562 101.532) (width 0.381) (layer B.Cu) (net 27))
 (segment (start 171.978 93.218) (end 171.978 89.555) (width 0.381) (layer B.Cu) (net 26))
 (segment (start 171.831 89.408) (end 170.248 89.408) (width 0.381) (layer B.Cu) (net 26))
 (segment (start 171.978 89.555) (end 171.831 89.408) (width 0.381) (layer B.Cu) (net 26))
 (segment (start 207.518 96.012) (end 207.518 90.932) (width 0.381) (layer B.Cu) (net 33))
 (segment (start 193.548 77.978) (end 189.813 77.978) (width 0.381) (layer B.Cu) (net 23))
 (segment (start 189.813 77.978) (end 179.653 67.818) (width 0.381) (layer B.Cu) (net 23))
 (segment (start 170.248 88.458) (end 170.248 85.958) (width 0.381) (layer B.Cu) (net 23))
 (segment (start 170.248 85.958) (end 170.608 85.598) (width 0.381) (layer B.Cu) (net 23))
 (segment (start 166.803 67.818) (end 166.803 84.507) (width 0.381) (layer B.Cu) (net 23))
 (segment (start 167.894 85.598) (end 170.608 85.598) (width 0.381) (layer B.Cu) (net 23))
 (segment (start 166.803 84.507) (end 167.894 85.598) (width 0.381) (layer B.Cu) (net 23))
 (segment (start 166.803 67.818) (end 179.653 67.818) (width 0.381) (layer B.Cu) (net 23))
 (segment (start 176.282 107.832) (end 176.282 106.706) (width 0.381) (layer B.Cu) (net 25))
 (segment (start 176.282 106.706) (end 173.482 103.906) (width 0.381) (layer B.Cu) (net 25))
 (segment (start 165.1 104.394) (end 172.994 104.394) (width 0.381) (layer B.Cu) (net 25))
 (segment (start 172.994 104.394) (end 173.482 103.906) (width 0.381) (layer B.Cu) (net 25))
 (segment (start 190.738 84.455) (end 190.738 86.598) (width 0.381) (layer B.Cu) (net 29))
 (segment (start 190.738 86.598) (end 190.754 86.614) (width 0.381) (layer B.Cu) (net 29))
 (segment (start 184.168 84.473) (end 190.72 84.473) (width 0.381) (layer B.Cu) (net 29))
 (segment (start 190.72 84.473) (end 190.738 84.455) (width 0.381) (layer B.Cu) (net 29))
 (segment (start 180.068 84.473) (end 180.993 84.473) (width 0.381) (layer B.Cu) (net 28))
 (segment (start 183.243 86.723) (end 184.168 86.723) (width 0.381) (layer B.Cu) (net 28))
 (segment (start 180.993 84.473) (end 183.243 86.723) (width 0.381) (layer B.Cu) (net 28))
 (segment (start 180.068 84.473) (end 174.433 84.473) (width 0.381) (layer B.Cu) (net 28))
 (segment (start 174.433 84.473) (end 173.308 85.598) (width 0.381) (layer B.Cu) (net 28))
 (segment (start 173.668 88.458) (end 173.668 85.958) (width 0.381) (layer B.Cu) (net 28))
 (segment (start 173.668 85.958) (end 173.308 85.598) (width 0.381) (layer B.Cu) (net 28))
 (segment (start 185.975 88.9) (end 180.594 88.9) (width 0.381) (layer B.Cu) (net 30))
 (segment (start 180.068 88.374) (end 180.068 86.723) (width 0.381) (layer B.Cu) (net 30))
 (segment (start 180.594 88.9) (end 180.068 88.374) (width 0.381) (layer B.Cu) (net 30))
 (segment (start 165.1 90.424) (end 170.182 90.424) (width 0.381) (layer B.Cu) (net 32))
 (segment (start 170.182 90.424) (end 170.248 90.358) (width 0.381) (layer B.Cu) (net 32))
 (segment (start 188.675 88.9) (end 188.675 85.468) (width 0.381) (layer B.Cu) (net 31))
 (segment (start 188.675 85.468) (end 188.738 85.405) (width 0.381) (layer B.Cu) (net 31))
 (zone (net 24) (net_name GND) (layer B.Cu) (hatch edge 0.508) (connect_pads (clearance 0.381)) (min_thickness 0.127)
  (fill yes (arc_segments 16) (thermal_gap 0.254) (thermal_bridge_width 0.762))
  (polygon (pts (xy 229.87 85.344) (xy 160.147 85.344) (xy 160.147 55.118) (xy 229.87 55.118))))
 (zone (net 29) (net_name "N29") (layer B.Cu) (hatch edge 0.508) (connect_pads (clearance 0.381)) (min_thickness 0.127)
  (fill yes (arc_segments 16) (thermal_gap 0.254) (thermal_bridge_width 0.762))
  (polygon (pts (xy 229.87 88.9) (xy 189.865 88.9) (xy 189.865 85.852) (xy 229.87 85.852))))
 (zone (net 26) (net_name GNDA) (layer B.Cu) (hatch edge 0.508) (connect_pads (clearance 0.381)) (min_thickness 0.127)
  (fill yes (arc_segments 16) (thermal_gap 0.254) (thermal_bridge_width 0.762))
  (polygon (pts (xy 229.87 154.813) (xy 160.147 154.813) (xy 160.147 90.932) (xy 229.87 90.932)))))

